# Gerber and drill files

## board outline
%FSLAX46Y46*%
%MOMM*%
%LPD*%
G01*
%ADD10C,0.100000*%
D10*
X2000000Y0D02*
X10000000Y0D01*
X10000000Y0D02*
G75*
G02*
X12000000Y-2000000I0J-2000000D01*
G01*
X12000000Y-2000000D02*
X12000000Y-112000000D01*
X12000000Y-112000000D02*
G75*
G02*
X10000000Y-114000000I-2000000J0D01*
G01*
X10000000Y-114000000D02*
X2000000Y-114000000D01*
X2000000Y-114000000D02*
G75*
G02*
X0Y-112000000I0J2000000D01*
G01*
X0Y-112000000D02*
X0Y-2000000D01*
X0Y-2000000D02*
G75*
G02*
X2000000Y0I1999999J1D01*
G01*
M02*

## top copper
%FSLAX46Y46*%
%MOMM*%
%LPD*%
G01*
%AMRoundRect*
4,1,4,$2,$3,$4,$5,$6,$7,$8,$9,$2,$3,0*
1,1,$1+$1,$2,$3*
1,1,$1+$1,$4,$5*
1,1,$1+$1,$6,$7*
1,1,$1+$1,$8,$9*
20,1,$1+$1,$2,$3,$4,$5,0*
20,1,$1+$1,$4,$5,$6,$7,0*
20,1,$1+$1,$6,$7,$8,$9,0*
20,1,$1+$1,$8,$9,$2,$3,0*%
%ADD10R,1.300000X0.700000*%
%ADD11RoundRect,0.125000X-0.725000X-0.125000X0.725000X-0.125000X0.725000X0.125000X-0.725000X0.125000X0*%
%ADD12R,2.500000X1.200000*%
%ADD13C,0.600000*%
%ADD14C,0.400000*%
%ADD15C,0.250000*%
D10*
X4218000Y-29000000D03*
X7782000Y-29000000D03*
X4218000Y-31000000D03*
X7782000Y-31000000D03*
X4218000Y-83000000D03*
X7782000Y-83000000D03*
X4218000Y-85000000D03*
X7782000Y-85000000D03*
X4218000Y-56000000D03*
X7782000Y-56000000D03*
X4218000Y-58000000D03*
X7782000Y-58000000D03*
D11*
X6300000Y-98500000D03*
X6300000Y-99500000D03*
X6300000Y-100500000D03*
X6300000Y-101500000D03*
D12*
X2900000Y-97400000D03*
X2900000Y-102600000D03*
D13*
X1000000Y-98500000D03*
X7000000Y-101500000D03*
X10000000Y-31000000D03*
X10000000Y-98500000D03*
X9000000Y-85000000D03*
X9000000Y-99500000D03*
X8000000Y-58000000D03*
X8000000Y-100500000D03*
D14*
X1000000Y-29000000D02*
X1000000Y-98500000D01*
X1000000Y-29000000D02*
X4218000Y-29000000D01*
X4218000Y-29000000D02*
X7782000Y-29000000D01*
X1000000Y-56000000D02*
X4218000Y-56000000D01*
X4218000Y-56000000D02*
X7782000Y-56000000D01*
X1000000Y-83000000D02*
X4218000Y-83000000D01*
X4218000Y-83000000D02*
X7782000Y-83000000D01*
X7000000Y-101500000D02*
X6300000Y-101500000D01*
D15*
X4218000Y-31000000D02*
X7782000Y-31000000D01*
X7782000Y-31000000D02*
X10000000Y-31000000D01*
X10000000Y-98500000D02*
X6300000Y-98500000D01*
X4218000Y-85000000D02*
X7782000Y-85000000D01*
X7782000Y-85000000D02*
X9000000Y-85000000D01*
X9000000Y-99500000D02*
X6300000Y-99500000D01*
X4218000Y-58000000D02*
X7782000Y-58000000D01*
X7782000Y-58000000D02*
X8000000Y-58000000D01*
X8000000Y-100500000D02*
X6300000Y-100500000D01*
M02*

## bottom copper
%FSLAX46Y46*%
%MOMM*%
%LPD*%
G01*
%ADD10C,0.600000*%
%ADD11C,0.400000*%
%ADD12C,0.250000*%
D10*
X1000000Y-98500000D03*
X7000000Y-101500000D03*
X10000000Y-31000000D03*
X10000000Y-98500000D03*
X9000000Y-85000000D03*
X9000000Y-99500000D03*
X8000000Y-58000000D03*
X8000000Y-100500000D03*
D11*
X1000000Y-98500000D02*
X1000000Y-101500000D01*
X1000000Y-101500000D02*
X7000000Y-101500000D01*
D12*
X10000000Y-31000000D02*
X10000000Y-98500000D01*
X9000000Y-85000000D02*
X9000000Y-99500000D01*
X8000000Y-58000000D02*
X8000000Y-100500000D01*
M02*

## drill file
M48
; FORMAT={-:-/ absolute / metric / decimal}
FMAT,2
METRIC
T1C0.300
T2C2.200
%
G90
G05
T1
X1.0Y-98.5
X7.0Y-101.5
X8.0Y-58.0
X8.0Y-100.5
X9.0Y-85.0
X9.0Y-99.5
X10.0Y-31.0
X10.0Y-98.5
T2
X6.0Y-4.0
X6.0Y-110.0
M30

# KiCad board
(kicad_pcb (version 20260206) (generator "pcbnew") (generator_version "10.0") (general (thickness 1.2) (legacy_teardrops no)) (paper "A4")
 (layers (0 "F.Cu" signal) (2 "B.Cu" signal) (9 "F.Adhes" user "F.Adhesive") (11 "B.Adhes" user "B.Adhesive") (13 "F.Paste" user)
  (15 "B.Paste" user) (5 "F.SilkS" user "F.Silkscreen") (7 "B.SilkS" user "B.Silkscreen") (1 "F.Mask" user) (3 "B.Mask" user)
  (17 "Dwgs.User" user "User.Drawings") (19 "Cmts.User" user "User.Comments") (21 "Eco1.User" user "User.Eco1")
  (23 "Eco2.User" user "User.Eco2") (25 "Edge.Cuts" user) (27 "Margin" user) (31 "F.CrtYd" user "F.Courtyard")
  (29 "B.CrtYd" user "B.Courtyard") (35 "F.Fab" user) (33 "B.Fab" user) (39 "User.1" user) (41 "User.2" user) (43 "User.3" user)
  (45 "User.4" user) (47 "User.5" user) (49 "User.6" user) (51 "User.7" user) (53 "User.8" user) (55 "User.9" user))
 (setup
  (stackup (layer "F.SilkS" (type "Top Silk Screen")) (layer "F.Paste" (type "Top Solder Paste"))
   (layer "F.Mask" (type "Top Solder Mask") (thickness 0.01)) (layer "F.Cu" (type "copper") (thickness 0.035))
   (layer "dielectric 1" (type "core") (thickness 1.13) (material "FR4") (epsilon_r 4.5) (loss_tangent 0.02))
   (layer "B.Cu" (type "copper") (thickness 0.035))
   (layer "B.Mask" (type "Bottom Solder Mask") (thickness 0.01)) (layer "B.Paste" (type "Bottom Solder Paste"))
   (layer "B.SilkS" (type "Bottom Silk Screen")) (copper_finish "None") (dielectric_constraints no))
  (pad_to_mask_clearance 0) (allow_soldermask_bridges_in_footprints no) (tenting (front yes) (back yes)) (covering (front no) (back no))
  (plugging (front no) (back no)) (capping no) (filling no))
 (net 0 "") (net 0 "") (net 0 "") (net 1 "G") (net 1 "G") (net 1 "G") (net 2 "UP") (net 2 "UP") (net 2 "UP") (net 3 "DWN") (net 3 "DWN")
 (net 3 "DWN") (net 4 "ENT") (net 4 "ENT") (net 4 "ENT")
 (gr_line (start 2 0) (end 10 0) (stroke (width 0.1) (type default)) (layer "Edge.Cuts"))
 (gr_arc (start 10 0) (mid 11.414214 0.585786) (end 12 2) (stroke (width 0.1) (type default)) (layer "Edge.Cuts"))
 (gr_line (start 12 2) (end 12 112) (stroke (width 0.1) (type default)) (layer "Edge.Cuts"))
 (gr_arc (start 12 112) (mid 11.414214 113.414214) (end 10 114) (stroke (width 0.1) (type default)) (layer "Edge.Cuts"))
 (gr_line (start 10 114) (end 2 114) (stroke (width 0.1) (type default)) (layer "Edge.Cuts"))
 (gr_arc (start 2 114) (mid 0.585786 113.414214) (end 0 112) (stroke (width 0.1) (type default)) (layer "Edge.Cuts"))
 (gr_line (start 0 112) (end 0 2) (stroke (width 0.1) (type default)) (layer "Edge.Cuts"))
 (gr_arc (start 0 2) (mid 0.585786 0.585786) (end 2 0) (stroke (width 0.1) (type default)) (layer "Edge.Cuts"))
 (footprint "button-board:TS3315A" (layer "F.Cu") (at 6 30)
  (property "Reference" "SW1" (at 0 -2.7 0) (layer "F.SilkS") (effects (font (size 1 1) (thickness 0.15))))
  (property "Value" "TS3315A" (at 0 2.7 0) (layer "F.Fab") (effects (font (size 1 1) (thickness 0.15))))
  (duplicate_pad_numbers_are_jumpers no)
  (pad "1" smd rect (at -1.782 -1.0) (size 1.3 0.7) (layers "F.Cu" "F.Mask" "F.Paste") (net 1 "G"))
  (pad "1" smd rect (at 1.782 -1.0) (size 1.3 0.7) (layers "F.Cu" "F.Mask" "F.Paste") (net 1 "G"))
  (pad "2" smd rect (at -1.782 1.0) (size 1.3 0.7) (layers "F.Cu" "F.Mask" "F.Paste") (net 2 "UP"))
  (pad "2" smd rect (at 1.782 1.0) (size 1.3 0.7) (layers "F.Cu" "F.Mask" "F.Paste") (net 2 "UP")))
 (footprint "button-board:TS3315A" (layer "F.Cu") (at 6 84)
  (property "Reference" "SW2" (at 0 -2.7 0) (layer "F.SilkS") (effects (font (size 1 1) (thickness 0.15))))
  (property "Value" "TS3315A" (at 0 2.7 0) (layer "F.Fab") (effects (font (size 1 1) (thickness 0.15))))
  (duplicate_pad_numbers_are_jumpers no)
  (pad "1" smd rect (at -1.782 -1.0) (size 1.3 0.7) (layers "F.Cu" "F.Mask" "F.Paste") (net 1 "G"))
  (pad "1" smd rect (at 1.782 -1.0) (size 1.3 0.7) (layers "F.Cu" "F.Mask" "F.Paste") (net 1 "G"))
  (pad "2" smd rect (at -1.782 1.0) (size 1.3 0.7) (layers "F.Cu" "F.Mask" "F.Paste") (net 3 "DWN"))
  (pad "2" smd rect (at 1.782 1.0) (size 1.3 0.7) (layers "F.Cu" "F.Mask" "F.Paste") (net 3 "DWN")))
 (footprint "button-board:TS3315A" (layer "F.Cu") (at 6 57)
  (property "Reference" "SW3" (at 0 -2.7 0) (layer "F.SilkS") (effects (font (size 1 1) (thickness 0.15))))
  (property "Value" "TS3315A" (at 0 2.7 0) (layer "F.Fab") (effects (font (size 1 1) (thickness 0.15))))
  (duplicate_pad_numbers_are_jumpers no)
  (pad "1" smd rect (at -1.782 -1.0) (size 1.3 0.7) (layers "F.Cu" "F.Mask" "F.Paste") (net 1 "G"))
  (pad "1" smd rect (at 1.782 -1.0) (size 1.3 0.7) (layers "F.Cu" "F.Mask" "F.Paste") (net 1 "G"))
  (pad "2" smd rect (at -1.782 1.0) (size 1.3 0.7) (layers "F.Cu" "F.Mask" "F.Paste") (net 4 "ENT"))
  (pad "2" smd rect (at 1.782 1.0) (size 1.3 0.7) (layers "F.Cu" "F.Mask" "F.Paste") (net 4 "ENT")))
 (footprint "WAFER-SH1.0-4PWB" (layer "F.Cu") (at 2 100)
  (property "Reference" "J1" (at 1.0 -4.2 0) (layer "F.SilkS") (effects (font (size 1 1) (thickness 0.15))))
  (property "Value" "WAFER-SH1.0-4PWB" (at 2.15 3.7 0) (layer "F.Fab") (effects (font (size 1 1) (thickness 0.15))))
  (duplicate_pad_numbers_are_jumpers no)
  (pad "1" smd roundrect (at 4.3 -1.5) (size 1.7 0.5) (layers "F.Cu" "F.Mask" "F.Paste") (roundrect_rratio 0.25) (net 2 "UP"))
  (pad "2" smd roundrect (at 4.3 -0.5) (size 1.7 0.5) (layers "F.Cu" "F.Mask" "F.Paste") (roundrect_rratio 0.25) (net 3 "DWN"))
  (pad "3" smd roundrect (at 4.3 0.5) (size 1.7 0.5) (layers "F.Cu" "F.Mask" "F.Paste") (roundrect_rratio 0.25) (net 4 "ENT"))
  (pad "4" smd roundrect (at 4.3 1.5) (size 1.7 0.5) (layers "F.Cu" "F.Mask" "F.Paste") (roundrect_rratio 0.25) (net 1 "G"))
  (pad "5" smd rect (at 0.9 -2.6) (size 2.5 1.2) (layers "F.Cu" "F.Mask" "F.Paste"))
  (pad "6" smd rect (at 0.9 2.6) (size 2.5 1.2) (layers "F.Cu" "F.Mask" "F.Paste")))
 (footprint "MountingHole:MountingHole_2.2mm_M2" (layer "F.Cu") (at 6 4) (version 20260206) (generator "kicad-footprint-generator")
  (layer "F.Cu")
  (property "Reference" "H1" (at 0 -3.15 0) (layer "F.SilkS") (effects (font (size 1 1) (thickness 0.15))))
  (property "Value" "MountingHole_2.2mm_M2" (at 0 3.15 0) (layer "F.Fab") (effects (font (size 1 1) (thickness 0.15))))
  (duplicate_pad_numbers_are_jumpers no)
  (pad "" np_thru_hole circle (at 0 0) (size 2.2 2.2) (drill 2.2) (layers "*.Cu" "*.Mask")))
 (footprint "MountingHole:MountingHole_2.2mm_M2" (layer "F.Cu") (at 6 110) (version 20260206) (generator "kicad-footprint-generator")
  (layer "F.Cu")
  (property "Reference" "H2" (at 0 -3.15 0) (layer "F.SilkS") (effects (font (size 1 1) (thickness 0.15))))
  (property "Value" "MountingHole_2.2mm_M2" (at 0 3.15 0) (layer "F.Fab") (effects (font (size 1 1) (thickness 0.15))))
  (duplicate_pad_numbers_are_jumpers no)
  (pad "" np_thru_hole circle (at 0 0) (size 2.2 2.2) (drill 2.2) (layers "*.Cu" "*.Mask")))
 (segment (start 1 29) (end 1 98.5) (width 0.4) (layer "F.Cu") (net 1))
 (segment (start 1 29) (end 4.218 29) (width 0.4) (layer "F.Cu") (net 1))
 (segment (start 4.218 29) (end 7.782 29) (width 0.4) (layer "F.Cu") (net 1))
 (segment (start 1 56) (end 4.218 56) (width 0.4) (layer "F.Cu") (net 1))
 (segment (start 4.218 56) (end 7.782 56) (width 0.4) (layer "F.Cu") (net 1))
 (segment (start 1 83) (end 4.218 83) (width 0.4) (layer "F.Cu") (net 1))
 (segment (start 4.218 83) (end 7.782 83) (width 0.4) (layer "F.Cu") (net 1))
 (via (at 1 98.5) (size 0.6) (drill 0.3) (layers "F.Cu" "B.Cu") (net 1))
 (segment (start 1 98.5) (end 1 101.5) (width 0.4) (layer "B.Cu") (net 1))
 (segment (start 1 101.5) (end 7.0 101.5) (width 0.4) (layer "B.Cu") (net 1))
 (via (at 7.0 101.5) (size 0.6) (drill 0.3) (layers "F.Cu" "B.Cu") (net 1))
 (segment (start 7.0 101.5) (end 6.3 101.5) (width 0.4) (layer "F.Cu") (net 1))
 (segment (start 4.218 31) (end 7.782 31) (width 0.25) (layer "F.Cu") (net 2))
 (segment (start 7.782 31) (end 10 31) (width 0.25) (layer "F.Cu") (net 2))
 (via (at 10 31) (size 0.6) (drill 0.3) (layers "F.Cu" "B.Cu") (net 2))
 (segment (start 10 31) (end 10 98.5) (width 0.25) (layer "B.Cu") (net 2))
 (via (at 10 98.5) (size 0.6) (drill 0.3) (layers "F.Cu" "B.Cu") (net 2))
 (segment (start 10 98.5) (end 6.3 98.5) (width 0.25) (layer "F.Cu") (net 2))
 (segment (start 4.218 85) (end 7.782 85) (width 0.25) (layer "F.Cu") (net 3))
 (segment (start 7.782 85) (end 9 85) (width 0.25) (layer "F.Cu") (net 3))
 (via (at 9 85) (size 0.6) (drill 0.3) (layers "F.Cu" "B.Cu") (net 3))
 (segment (start 9 85) (end 9 99.5) (width 0.25) (layer "B.Cu") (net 3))
 (via (at 9 99.5) (size 0.6) (drill 0.3) (layers "F.Cu" "B.Cu") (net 3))
 (segment (start 9 99.5) (end 6.3 99.5) (width 0.25) (layer "F.Cu") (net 3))
 (segment (start 4.218 58) (end 7.782 58) (width 0.25) (layer "F.Cu") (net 4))
 (segment (start 7.782 58) (end 8 58) (width 0.25) (layer "F.Cu") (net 4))
 (via (at 8 58) (size 0.6) (drill 0.3) (layers "F.Cu" "B.Cu") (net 4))
 (segment (start 8 58) (end 8 100.5) (width 0.25) (layer "B.Cu") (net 4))
 (via (at 8 100.5) (size 0.6) (drill 0.3) (layers "F.Cu" "B.Cu") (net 4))
 (segment (start 8 100.5) (end 6.3 100.5) (width 0.25) (layer "F.Cu") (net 4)))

